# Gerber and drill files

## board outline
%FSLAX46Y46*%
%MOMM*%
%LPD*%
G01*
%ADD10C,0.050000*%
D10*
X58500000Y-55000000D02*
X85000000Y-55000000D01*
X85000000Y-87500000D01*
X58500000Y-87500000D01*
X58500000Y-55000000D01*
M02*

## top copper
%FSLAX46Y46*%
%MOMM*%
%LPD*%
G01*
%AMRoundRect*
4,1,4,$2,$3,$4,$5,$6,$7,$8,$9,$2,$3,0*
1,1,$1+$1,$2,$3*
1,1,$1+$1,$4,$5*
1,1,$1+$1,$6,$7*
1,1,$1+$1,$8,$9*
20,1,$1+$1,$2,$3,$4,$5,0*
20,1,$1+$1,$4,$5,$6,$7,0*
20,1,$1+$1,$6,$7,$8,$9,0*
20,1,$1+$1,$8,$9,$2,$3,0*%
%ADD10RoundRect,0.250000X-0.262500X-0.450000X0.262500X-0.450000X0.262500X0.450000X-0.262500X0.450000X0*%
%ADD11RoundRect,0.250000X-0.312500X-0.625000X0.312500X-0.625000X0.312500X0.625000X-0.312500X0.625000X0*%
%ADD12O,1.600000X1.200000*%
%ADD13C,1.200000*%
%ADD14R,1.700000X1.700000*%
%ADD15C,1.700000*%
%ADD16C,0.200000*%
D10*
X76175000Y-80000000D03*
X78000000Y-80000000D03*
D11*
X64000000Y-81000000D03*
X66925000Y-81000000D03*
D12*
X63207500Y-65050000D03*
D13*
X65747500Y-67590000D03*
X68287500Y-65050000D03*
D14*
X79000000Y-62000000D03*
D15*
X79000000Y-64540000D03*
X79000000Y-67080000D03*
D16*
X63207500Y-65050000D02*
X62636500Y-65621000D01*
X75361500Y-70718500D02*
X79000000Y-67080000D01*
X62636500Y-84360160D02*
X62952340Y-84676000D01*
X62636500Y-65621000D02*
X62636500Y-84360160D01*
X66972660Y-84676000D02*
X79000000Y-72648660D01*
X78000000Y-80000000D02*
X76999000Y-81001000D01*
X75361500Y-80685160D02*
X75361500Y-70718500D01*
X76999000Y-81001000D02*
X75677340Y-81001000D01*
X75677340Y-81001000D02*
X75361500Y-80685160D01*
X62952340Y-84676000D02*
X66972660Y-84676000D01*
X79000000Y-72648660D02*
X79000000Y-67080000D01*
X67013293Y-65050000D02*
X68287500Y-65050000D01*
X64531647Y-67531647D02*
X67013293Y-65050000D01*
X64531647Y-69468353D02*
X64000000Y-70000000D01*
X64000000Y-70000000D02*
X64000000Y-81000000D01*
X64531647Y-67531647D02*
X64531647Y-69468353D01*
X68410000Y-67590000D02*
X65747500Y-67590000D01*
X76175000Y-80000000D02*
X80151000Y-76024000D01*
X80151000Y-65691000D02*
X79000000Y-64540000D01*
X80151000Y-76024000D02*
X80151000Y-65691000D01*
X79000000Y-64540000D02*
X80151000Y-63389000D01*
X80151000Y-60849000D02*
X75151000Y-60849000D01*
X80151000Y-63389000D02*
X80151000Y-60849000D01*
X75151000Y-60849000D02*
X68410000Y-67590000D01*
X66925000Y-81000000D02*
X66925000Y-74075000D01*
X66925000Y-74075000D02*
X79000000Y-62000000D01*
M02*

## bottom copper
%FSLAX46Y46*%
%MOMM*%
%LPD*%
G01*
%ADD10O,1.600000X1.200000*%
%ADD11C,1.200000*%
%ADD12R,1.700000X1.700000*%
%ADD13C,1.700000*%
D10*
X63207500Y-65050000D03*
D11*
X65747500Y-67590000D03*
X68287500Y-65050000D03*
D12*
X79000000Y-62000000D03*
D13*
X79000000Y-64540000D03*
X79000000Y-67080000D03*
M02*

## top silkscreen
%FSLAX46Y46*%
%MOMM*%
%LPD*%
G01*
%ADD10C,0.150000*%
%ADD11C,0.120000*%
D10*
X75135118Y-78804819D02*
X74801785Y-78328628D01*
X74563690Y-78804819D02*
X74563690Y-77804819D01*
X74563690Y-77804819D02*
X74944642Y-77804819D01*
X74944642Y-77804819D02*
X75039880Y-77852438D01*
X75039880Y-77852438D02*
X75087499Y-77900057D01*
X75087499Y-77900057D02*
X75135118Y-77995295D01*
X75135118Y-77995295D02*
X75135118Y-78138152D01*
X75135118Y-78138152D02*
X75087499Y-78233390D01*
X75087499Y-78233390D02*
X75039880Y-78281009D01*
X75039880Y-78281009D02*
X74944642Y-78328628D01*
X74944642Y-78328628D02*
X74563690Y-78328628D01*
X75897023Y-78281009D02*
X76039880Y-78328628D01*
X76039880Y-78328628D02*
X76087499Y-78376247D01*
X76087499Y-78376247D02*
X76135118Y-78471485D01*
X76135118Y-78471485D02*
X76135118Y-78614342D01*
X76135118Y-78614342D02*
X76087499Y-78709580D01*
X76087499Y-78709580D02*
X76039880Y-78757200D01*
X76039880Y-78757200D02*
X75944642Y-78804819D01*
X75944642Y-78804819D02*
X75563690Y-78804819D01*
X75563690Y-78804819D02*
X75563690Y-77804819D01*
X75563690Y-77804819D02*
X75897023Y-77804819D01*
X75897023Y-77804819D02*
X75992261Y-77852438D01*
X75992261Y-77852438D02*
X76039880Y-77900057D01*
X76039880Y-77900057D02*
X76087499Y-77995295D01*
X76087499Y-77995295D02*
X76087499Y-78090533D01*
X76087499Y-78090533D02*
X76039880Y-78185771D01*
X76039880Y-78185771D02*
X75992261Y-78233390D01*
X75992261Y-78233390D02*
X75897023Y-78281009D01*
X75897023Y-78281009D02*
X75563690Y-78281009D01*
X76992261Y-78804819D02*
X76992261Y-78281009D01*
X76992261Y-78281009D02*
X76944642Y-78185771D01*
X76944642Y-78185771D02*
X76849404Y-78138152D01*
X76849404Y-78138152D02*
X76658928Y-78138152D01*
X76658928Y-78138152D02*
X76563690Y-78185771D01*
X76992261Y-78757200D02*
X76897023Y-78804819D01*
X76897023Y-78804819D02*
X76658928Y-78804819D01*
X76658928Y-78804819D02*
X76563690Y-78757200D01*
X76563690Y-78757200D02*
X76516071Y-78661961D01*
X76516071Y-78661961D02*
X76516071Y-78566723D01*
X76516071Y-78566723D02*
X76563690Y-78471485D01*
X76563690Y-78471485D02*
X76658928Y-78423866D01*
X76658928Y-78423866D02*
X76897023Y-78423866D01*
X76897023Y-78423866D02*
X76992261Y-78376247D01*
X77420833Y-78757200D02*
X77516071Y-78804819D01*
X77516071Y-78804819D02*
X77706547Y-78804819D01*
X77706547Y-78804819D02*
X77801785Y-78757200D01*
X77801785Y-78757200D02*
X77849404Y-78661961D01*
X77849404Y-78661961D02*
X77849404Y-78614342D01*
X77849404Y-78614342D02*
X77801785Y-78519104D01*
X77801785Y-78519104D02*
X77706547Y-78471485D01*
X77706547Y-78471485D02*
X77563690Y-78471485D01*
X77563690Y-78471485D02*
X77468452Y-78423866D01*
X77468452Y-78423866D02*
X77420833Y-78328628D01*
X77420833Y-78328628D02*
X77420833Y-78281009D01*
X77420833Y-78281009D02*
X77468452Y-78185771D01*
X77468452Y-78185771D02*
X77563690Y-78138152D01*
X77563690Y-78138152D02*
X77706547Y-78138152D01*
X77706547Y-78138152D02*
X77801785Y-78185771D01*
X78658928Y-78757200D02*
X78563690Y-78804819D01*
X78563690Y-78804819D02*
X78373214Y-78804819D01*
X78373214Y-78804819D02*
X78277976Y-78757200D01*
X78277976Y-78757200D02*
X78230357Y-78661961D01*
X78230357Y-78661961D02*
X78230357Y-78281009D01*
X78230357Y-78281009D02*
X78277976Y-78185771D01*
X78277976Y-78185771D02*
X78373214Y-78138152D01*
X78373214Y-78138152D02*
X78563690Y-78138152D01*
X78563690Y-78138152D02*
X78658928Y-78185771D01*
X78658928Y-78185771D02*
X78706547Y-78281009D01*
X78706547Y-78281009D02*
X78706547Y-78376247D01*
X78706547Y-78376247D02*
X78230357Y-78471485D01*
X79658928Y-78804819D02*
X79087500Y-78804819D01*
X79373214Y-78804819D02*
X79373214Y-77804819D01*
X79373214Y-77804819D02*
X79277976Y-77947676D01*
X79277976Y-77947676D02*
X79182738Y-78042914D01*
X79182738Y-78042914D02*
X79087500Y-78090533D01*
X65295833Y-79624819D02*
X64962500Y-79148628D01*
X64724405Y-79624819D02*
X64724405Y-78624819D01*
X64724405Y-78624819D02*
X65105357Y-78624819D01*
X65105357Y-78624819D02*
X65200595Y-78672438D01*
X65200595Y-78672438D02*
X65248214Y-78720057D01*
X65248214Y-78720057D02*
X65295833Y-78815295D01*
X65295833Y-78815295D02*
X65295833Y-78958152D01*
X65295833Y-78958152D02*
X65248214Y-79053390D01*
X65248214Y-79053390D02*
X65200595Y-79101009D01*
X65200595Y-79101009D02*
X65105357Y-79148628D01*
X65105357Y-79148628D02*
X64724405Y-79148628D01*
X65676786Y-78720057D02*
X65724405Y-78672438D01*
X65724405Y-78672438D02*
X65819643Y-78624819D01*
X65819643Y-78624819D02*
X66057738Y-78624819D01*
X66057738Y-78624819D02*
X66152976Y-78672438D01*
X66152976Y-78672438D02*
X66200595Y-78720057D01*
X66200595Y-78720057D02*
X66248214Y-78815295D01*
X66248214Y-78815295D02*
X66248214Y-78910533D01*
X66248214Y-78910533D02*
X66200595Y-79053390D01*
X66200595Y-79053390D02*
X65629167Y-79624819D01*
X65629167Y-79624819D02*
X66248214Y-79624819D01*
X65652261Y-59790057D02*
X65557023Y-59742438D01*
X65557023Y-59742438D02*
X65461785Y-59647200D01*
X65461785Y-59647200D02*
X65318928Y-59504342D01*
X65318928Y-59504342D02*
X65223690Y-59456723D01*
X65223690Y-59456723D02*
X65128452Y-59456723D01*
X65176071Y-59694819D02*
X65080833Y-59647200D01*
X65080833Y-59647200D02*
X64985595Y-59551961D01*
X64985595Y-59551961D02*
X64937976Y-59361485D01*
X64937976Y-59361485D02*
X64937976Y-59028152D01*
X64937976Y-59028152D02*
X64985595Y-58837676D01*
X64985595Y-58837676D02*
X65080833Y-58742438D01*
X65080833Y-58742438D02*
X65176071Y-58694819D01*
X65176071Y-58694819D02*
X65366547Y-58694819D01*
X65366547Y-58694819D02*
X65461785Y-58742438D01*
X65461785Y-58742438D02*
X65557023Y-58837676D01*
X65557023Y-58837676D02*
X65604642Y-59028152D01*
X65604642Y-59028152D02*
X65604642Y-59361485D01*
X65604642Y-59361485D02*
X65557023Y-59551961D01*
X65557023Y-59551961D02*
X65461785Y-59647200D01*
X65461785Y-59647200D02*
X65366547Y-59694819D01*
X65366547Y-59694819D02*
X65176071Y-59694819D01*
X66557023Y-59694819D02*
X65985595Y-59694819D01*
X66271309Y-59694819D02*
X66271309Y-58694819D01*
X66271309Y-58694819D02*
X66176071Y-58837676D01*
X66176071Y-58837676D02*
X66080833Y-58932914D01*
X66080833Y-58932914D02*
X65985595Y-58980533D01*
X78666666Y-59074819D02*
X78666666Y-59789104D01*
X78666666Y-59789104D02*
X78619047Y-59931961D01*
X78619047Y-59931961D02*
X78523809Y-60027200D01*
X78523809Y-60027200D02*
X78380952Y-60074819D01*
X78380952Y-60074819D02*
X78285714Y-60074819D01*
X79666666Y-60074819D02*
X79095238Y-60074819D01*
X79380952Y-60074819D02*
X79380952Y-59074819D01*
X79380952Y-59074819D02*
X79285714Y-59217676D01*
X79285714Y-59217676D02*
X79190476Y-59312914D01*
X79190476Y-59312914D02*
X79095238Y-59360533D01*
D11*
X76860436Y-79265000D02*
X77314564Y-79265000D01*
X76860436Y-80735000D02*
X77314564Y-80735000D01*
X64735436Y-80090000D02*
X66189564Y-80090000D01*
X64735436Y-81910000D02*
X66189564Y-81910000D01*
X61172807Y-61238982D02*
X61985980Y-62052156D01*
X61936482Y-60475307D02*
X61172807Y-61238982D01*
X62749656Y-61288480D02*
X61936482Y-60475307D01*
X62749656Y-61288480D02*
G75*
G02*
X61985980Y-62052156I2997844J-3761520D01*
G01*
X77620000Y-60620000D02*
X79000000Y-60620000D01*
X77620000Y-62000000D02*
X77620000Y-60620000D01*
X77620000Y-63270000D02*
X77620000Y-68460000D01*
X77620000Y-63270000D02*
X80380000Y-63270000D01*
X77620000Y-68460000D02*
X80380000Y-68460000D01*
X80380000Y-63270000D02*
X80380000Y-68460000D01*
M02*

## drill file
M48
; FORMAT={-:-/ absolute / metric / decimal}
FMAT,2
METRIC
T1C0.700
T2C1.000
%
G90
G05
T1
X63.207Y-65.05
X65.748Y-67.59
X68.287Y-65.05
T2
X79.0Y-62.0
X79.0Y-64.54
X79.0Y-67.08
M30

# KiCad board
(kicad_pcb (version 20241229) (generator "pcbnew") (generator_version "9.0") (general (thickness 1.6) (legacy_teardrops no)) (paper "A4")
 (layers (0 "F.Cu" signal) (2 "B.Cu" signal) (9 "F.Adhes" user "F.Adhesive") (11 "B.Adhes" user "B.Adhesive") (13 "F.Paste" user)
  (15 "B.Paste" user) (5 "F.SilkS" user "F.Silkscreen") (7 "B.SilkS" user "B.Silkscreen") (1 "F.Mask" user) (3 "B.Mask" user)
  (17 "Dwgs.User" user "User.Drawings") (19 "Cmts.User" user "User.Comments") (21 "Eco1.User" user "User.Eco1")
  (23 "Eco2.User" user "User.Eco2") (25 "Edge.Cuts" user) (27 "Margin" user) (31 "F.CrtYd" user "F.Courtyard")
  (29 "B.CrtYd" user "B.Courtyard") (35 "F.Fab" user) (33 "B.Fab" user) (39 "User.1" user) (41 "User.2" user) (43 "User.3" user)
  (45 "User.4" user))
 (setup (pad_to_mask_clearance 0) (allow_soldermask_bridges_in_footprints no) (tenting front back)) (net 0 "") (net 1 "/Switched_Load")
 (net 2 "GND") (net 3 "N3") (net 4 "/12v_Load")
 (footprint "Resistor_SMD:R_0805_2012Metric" (layer "F.Cu") (at 77.0875 80)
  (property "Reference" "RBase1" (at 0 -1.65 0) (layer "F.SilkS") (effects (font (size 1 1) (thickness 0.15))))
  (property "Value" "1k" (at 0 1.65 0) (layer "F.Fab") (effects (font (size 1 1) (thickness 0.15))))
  (fp_line (start -0.227064 -0.735) (end 0.227064 -0.735) (stroke (width 0.12) (type solid)) (layer "F.SilkS"))
  (fp_line (start -0.227064 0.735) (end 0.227064 0.735) (stroke (width 0.12) (type solid)) (layer "F.SilkS"))
  (pad "1" smd roundrect (at -0.9125 0) (size 1.025 1.4) (layers "F.Cu" "F.Mask" "F.Paste") (roundrect_rratio 0.243902)
   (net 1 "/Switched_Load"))
  (pad "2" smd roundrect (at 0.9125 0) (size 1.025 1.4) (layers "F.Cu" "F.Mask" "F.Paste") (roundrect_rratio 0.243902) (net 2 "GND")))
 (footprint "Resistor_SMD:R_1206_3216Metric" (layer "F.Cu") (at 65.4625 81)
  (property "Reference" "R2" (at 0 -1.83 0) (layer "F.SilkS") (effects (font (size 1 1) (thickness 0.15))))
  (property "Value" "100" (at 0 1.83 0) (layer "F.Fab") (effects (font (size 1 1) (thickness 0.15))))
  (fp_line (start -0.727064 -0.91) (end 0.727064 -0.91) (stroke (width 0.12) (type solid)) (layer "F.SilkS"))
  (fp_line (start -0.727064 0.91) (end 0.727064 0.91) (stroke (width 0.12) (type solid)) (layer "F.SilkS"))
  (pad "1" smd roundrect (at -1.4625 0) (size 1.125 1.75) (layers "F.Cu" "F.Mask" "F.Paste") (roundrect_rratio 0.222222) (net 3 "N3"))
  (pad "2" smd roundrect (at 1.4625 0) (size 1.125 1.75) (layers "F.Cu" "F.Mask" "F.Paste") (roundrect_rratio 0.222222) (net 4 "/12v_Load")))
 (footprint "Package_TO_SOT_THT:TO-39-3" (layer "F.Cu") (at 63.2075 65.05)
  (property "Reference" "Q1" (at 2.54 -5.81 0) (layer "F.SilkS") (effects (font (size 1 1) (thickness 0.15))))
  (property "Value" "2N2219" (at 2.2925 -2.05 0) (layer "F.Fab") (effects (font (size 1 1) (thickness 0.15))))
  (fp_line (start -2.034693 -3.811018) (end -1.22152 -2.997844) (stroke (width 0.12) (type solid)) (layer "F.SilkS"))
  (fp_line (start -1.271018 -4.574693) (end -2.034693 -3.811018) (stroke (width 0.12) (type solid)) (layer "F.SilkS"))
  (fp_line (start -0.457844 -3.76152) (end -1.271018 -4.574693) (stroke (width 0.12) (type solid)) (layer "F.SilkS"))
  (fp_arc (start -0.457844 -3.76152) (mid 5.941184 3.401184) (end -1.22152 -2.997844) (stroke (width 0.12) (type solid)) (layer "F.SilkS"))
  (pad "1" thru_hole oval (at 0 0) (size 1.6 1.2) (drill 0.7) (layers "*.Cu" "*.Mask") (remove_unused_layers no) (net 2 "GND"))
  (pad "2" thru_hole circle (at 2.54 2.54) (size 1.2 1.2) (drill 0.7) (layers "*.Cu" "*.Mask") (remove_unused_layers no)
   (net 1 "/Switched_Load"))
  (pad "3" thru_hole circle (at 5.08 0) (size 1.2 1.2) (drill 0.7) (layers "*.Cu" "*.Mask") (remove_unused_layers no) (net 3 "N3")))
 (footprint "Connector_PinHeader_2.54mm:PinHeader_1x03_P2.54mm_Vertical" (layer "F.Cu") (at 79 62)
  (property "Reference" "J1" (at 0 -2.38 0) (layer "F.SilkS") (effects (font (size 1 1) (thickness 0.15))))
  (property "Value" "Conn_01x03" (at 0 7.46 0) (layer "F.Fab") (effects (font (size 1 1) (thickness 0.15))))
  (fp_line (start -1.38 -1.38) (end 0 -1.38) (stroke (width 0.12) (type solid)) (layer "F.SilkS"))
  (fp_line (start -1.38 0) (end -1.38 -1.38) (stroke (width 0.12) (type solid)) (layer "F.SilkS"))
  (fp_line (start -1.38 1.27) (end -1.38 6.46) (stroke (width 0.12) (type solid)) (layer "F.SilkS"))
  (fp_line (start -1.38 1.27) (end 1.38 1.27) (stroke (width 0.12) (type solid)) (layer "F.SilkS"))
  (fp_line (start -1.38 6.46) (end 1.38 6.46) (stroke (width 0.12) (type solid)) (layer "F.SilkS"))
  (fp_line (start 1.38 1.27) (end 1.38 6.46) (stroke (width 0.12) (type solid)) (layer "F.SilkS"))
  (pad "1" thru_hole rect (at 0 0) (size 1.7 1.7) (drill 1) (layers "*.Cu" "*.Mask") (remove_unused_layers no) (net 4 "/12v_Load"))
  (pad "2" thru_hole circle (at 0 2.54) (size 1.7 1.7) (drill 1) (layers "*.Cu" "*.Mask") (remove_unused_layers no) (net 1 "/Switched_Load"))
  (pad "3" thru_hole circle (at 0 5.08) (size 1.7 1.7) (drill 1) (layers "*.Cu" "*.Mask") (remove_unused_layers no) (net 2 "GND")))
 (gr_rect (start 58.5 55) (end 85 87.5) (stroke (width 0.05) (type default)) (fill no) (layer "Edge.Cuts"))
 (segment (start 63.2075 65.05) (end 62.6365 65.621) (width 0.2) (layer "F.Cu") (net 2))
 (segment (start 75.3615 70.7185) (end 79 67.08) (width 0.2) (layer "F.Cu") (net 2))
 (segment (start 62.6365 84.36016) (end 62.95234 84.676) (width 0.2) (layer "F.Cu") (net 2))
 (segment (start 62.6365 65.621) (end 62.6365 84.36016) (width 0.2) (layer "F.Cu") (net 2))
 (segment (start 66.97266 84.676) (end 79 72.64866) (width 0.2) (layer "F.Cu") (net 2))
 (segment (start 78 80) (end 76.999 81.001) (width 0.2) (layer "F.Cu") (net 2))
 (segment (start 75.3615 80.68516) (end 75.3615 70.7185) (width 0.2) (layer "F.Cu") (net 2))
 (segment (start 76.999 81.001) (end 75.67734 81.001) (width 0.2) (layer "F.Cu") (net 2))
 (segment (start 75.67734 81.001) (end 75.3615 80.68516) (width 0.2) (layer "F.Cu") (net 2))
 (segment (start 62.95234 84.676) (end 66.97266 84.676) (width 0.2) (layer "F.Cu") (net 2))
 (segment (start 79 72.64866) (end 79 67.08) (width 0.2) (layer "F.Cu") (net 2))
 (segment (start 67.013293 65.05) (end 68.2875 65.05) (width 0.2) (layer "F.Cu") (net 3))
 (segment (start 64.531647 67.531647) (end 67.013293 65.05) (width 0.2) (layer "F.Cu") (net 3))
 (segment (start 64.531647 69.468353) (end 64 70) (width 0.2) (layer "F.Cu") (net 3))
 (segment (start 64 70) (end 64 81) (width 0.2) (layer "F.Cu") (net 3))
 (segment (start 64.531647 67.531647) (end 64.531647 69.468353) (width 0.2) (layer "F.Cu") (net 3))
 (segment (start 68.41 67.59) (end 65.7475 67.59) (width 0.2) (layer "F.Cu") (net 1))
 (segment (start 76.175 80) (end 80.151 76.024) (width 0.2) (layer "F.Cu") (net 1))
 (segment (start 80.151 65.691) (end 79 64.54) (width 0.2) (layer "F.Cu") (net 1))
 (segment (start 80.151 76.024) (end 80.151 65.691) (width 0.2) (layer "F.Cu") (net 1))
 (segment (start 79 64.54) (end 80.151 63.389) (width 0.2) (layer "F.Cu") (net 1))
 (segment (start 80.151 60.849) (end 75.151 60.849) (width 0.2) (layer "F.Cu") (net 1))
 (segment (start 80.151 63.389) (end 80.151 60.849) (width 0.2) (layer "F.Cu") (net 1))
 (segment (start 75.151 60.849) (end 68.41 67.59) (width 0.2) (layer "F.Cu") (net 1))
 (segment (start 66.925 81) (end 66.925 74.075) (width 0.2) (layer "F.Cu") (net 4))
 (segment (start 66.925 74.075) (end 79 62) (width 0.2) (layer "F.Cu") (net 4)))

